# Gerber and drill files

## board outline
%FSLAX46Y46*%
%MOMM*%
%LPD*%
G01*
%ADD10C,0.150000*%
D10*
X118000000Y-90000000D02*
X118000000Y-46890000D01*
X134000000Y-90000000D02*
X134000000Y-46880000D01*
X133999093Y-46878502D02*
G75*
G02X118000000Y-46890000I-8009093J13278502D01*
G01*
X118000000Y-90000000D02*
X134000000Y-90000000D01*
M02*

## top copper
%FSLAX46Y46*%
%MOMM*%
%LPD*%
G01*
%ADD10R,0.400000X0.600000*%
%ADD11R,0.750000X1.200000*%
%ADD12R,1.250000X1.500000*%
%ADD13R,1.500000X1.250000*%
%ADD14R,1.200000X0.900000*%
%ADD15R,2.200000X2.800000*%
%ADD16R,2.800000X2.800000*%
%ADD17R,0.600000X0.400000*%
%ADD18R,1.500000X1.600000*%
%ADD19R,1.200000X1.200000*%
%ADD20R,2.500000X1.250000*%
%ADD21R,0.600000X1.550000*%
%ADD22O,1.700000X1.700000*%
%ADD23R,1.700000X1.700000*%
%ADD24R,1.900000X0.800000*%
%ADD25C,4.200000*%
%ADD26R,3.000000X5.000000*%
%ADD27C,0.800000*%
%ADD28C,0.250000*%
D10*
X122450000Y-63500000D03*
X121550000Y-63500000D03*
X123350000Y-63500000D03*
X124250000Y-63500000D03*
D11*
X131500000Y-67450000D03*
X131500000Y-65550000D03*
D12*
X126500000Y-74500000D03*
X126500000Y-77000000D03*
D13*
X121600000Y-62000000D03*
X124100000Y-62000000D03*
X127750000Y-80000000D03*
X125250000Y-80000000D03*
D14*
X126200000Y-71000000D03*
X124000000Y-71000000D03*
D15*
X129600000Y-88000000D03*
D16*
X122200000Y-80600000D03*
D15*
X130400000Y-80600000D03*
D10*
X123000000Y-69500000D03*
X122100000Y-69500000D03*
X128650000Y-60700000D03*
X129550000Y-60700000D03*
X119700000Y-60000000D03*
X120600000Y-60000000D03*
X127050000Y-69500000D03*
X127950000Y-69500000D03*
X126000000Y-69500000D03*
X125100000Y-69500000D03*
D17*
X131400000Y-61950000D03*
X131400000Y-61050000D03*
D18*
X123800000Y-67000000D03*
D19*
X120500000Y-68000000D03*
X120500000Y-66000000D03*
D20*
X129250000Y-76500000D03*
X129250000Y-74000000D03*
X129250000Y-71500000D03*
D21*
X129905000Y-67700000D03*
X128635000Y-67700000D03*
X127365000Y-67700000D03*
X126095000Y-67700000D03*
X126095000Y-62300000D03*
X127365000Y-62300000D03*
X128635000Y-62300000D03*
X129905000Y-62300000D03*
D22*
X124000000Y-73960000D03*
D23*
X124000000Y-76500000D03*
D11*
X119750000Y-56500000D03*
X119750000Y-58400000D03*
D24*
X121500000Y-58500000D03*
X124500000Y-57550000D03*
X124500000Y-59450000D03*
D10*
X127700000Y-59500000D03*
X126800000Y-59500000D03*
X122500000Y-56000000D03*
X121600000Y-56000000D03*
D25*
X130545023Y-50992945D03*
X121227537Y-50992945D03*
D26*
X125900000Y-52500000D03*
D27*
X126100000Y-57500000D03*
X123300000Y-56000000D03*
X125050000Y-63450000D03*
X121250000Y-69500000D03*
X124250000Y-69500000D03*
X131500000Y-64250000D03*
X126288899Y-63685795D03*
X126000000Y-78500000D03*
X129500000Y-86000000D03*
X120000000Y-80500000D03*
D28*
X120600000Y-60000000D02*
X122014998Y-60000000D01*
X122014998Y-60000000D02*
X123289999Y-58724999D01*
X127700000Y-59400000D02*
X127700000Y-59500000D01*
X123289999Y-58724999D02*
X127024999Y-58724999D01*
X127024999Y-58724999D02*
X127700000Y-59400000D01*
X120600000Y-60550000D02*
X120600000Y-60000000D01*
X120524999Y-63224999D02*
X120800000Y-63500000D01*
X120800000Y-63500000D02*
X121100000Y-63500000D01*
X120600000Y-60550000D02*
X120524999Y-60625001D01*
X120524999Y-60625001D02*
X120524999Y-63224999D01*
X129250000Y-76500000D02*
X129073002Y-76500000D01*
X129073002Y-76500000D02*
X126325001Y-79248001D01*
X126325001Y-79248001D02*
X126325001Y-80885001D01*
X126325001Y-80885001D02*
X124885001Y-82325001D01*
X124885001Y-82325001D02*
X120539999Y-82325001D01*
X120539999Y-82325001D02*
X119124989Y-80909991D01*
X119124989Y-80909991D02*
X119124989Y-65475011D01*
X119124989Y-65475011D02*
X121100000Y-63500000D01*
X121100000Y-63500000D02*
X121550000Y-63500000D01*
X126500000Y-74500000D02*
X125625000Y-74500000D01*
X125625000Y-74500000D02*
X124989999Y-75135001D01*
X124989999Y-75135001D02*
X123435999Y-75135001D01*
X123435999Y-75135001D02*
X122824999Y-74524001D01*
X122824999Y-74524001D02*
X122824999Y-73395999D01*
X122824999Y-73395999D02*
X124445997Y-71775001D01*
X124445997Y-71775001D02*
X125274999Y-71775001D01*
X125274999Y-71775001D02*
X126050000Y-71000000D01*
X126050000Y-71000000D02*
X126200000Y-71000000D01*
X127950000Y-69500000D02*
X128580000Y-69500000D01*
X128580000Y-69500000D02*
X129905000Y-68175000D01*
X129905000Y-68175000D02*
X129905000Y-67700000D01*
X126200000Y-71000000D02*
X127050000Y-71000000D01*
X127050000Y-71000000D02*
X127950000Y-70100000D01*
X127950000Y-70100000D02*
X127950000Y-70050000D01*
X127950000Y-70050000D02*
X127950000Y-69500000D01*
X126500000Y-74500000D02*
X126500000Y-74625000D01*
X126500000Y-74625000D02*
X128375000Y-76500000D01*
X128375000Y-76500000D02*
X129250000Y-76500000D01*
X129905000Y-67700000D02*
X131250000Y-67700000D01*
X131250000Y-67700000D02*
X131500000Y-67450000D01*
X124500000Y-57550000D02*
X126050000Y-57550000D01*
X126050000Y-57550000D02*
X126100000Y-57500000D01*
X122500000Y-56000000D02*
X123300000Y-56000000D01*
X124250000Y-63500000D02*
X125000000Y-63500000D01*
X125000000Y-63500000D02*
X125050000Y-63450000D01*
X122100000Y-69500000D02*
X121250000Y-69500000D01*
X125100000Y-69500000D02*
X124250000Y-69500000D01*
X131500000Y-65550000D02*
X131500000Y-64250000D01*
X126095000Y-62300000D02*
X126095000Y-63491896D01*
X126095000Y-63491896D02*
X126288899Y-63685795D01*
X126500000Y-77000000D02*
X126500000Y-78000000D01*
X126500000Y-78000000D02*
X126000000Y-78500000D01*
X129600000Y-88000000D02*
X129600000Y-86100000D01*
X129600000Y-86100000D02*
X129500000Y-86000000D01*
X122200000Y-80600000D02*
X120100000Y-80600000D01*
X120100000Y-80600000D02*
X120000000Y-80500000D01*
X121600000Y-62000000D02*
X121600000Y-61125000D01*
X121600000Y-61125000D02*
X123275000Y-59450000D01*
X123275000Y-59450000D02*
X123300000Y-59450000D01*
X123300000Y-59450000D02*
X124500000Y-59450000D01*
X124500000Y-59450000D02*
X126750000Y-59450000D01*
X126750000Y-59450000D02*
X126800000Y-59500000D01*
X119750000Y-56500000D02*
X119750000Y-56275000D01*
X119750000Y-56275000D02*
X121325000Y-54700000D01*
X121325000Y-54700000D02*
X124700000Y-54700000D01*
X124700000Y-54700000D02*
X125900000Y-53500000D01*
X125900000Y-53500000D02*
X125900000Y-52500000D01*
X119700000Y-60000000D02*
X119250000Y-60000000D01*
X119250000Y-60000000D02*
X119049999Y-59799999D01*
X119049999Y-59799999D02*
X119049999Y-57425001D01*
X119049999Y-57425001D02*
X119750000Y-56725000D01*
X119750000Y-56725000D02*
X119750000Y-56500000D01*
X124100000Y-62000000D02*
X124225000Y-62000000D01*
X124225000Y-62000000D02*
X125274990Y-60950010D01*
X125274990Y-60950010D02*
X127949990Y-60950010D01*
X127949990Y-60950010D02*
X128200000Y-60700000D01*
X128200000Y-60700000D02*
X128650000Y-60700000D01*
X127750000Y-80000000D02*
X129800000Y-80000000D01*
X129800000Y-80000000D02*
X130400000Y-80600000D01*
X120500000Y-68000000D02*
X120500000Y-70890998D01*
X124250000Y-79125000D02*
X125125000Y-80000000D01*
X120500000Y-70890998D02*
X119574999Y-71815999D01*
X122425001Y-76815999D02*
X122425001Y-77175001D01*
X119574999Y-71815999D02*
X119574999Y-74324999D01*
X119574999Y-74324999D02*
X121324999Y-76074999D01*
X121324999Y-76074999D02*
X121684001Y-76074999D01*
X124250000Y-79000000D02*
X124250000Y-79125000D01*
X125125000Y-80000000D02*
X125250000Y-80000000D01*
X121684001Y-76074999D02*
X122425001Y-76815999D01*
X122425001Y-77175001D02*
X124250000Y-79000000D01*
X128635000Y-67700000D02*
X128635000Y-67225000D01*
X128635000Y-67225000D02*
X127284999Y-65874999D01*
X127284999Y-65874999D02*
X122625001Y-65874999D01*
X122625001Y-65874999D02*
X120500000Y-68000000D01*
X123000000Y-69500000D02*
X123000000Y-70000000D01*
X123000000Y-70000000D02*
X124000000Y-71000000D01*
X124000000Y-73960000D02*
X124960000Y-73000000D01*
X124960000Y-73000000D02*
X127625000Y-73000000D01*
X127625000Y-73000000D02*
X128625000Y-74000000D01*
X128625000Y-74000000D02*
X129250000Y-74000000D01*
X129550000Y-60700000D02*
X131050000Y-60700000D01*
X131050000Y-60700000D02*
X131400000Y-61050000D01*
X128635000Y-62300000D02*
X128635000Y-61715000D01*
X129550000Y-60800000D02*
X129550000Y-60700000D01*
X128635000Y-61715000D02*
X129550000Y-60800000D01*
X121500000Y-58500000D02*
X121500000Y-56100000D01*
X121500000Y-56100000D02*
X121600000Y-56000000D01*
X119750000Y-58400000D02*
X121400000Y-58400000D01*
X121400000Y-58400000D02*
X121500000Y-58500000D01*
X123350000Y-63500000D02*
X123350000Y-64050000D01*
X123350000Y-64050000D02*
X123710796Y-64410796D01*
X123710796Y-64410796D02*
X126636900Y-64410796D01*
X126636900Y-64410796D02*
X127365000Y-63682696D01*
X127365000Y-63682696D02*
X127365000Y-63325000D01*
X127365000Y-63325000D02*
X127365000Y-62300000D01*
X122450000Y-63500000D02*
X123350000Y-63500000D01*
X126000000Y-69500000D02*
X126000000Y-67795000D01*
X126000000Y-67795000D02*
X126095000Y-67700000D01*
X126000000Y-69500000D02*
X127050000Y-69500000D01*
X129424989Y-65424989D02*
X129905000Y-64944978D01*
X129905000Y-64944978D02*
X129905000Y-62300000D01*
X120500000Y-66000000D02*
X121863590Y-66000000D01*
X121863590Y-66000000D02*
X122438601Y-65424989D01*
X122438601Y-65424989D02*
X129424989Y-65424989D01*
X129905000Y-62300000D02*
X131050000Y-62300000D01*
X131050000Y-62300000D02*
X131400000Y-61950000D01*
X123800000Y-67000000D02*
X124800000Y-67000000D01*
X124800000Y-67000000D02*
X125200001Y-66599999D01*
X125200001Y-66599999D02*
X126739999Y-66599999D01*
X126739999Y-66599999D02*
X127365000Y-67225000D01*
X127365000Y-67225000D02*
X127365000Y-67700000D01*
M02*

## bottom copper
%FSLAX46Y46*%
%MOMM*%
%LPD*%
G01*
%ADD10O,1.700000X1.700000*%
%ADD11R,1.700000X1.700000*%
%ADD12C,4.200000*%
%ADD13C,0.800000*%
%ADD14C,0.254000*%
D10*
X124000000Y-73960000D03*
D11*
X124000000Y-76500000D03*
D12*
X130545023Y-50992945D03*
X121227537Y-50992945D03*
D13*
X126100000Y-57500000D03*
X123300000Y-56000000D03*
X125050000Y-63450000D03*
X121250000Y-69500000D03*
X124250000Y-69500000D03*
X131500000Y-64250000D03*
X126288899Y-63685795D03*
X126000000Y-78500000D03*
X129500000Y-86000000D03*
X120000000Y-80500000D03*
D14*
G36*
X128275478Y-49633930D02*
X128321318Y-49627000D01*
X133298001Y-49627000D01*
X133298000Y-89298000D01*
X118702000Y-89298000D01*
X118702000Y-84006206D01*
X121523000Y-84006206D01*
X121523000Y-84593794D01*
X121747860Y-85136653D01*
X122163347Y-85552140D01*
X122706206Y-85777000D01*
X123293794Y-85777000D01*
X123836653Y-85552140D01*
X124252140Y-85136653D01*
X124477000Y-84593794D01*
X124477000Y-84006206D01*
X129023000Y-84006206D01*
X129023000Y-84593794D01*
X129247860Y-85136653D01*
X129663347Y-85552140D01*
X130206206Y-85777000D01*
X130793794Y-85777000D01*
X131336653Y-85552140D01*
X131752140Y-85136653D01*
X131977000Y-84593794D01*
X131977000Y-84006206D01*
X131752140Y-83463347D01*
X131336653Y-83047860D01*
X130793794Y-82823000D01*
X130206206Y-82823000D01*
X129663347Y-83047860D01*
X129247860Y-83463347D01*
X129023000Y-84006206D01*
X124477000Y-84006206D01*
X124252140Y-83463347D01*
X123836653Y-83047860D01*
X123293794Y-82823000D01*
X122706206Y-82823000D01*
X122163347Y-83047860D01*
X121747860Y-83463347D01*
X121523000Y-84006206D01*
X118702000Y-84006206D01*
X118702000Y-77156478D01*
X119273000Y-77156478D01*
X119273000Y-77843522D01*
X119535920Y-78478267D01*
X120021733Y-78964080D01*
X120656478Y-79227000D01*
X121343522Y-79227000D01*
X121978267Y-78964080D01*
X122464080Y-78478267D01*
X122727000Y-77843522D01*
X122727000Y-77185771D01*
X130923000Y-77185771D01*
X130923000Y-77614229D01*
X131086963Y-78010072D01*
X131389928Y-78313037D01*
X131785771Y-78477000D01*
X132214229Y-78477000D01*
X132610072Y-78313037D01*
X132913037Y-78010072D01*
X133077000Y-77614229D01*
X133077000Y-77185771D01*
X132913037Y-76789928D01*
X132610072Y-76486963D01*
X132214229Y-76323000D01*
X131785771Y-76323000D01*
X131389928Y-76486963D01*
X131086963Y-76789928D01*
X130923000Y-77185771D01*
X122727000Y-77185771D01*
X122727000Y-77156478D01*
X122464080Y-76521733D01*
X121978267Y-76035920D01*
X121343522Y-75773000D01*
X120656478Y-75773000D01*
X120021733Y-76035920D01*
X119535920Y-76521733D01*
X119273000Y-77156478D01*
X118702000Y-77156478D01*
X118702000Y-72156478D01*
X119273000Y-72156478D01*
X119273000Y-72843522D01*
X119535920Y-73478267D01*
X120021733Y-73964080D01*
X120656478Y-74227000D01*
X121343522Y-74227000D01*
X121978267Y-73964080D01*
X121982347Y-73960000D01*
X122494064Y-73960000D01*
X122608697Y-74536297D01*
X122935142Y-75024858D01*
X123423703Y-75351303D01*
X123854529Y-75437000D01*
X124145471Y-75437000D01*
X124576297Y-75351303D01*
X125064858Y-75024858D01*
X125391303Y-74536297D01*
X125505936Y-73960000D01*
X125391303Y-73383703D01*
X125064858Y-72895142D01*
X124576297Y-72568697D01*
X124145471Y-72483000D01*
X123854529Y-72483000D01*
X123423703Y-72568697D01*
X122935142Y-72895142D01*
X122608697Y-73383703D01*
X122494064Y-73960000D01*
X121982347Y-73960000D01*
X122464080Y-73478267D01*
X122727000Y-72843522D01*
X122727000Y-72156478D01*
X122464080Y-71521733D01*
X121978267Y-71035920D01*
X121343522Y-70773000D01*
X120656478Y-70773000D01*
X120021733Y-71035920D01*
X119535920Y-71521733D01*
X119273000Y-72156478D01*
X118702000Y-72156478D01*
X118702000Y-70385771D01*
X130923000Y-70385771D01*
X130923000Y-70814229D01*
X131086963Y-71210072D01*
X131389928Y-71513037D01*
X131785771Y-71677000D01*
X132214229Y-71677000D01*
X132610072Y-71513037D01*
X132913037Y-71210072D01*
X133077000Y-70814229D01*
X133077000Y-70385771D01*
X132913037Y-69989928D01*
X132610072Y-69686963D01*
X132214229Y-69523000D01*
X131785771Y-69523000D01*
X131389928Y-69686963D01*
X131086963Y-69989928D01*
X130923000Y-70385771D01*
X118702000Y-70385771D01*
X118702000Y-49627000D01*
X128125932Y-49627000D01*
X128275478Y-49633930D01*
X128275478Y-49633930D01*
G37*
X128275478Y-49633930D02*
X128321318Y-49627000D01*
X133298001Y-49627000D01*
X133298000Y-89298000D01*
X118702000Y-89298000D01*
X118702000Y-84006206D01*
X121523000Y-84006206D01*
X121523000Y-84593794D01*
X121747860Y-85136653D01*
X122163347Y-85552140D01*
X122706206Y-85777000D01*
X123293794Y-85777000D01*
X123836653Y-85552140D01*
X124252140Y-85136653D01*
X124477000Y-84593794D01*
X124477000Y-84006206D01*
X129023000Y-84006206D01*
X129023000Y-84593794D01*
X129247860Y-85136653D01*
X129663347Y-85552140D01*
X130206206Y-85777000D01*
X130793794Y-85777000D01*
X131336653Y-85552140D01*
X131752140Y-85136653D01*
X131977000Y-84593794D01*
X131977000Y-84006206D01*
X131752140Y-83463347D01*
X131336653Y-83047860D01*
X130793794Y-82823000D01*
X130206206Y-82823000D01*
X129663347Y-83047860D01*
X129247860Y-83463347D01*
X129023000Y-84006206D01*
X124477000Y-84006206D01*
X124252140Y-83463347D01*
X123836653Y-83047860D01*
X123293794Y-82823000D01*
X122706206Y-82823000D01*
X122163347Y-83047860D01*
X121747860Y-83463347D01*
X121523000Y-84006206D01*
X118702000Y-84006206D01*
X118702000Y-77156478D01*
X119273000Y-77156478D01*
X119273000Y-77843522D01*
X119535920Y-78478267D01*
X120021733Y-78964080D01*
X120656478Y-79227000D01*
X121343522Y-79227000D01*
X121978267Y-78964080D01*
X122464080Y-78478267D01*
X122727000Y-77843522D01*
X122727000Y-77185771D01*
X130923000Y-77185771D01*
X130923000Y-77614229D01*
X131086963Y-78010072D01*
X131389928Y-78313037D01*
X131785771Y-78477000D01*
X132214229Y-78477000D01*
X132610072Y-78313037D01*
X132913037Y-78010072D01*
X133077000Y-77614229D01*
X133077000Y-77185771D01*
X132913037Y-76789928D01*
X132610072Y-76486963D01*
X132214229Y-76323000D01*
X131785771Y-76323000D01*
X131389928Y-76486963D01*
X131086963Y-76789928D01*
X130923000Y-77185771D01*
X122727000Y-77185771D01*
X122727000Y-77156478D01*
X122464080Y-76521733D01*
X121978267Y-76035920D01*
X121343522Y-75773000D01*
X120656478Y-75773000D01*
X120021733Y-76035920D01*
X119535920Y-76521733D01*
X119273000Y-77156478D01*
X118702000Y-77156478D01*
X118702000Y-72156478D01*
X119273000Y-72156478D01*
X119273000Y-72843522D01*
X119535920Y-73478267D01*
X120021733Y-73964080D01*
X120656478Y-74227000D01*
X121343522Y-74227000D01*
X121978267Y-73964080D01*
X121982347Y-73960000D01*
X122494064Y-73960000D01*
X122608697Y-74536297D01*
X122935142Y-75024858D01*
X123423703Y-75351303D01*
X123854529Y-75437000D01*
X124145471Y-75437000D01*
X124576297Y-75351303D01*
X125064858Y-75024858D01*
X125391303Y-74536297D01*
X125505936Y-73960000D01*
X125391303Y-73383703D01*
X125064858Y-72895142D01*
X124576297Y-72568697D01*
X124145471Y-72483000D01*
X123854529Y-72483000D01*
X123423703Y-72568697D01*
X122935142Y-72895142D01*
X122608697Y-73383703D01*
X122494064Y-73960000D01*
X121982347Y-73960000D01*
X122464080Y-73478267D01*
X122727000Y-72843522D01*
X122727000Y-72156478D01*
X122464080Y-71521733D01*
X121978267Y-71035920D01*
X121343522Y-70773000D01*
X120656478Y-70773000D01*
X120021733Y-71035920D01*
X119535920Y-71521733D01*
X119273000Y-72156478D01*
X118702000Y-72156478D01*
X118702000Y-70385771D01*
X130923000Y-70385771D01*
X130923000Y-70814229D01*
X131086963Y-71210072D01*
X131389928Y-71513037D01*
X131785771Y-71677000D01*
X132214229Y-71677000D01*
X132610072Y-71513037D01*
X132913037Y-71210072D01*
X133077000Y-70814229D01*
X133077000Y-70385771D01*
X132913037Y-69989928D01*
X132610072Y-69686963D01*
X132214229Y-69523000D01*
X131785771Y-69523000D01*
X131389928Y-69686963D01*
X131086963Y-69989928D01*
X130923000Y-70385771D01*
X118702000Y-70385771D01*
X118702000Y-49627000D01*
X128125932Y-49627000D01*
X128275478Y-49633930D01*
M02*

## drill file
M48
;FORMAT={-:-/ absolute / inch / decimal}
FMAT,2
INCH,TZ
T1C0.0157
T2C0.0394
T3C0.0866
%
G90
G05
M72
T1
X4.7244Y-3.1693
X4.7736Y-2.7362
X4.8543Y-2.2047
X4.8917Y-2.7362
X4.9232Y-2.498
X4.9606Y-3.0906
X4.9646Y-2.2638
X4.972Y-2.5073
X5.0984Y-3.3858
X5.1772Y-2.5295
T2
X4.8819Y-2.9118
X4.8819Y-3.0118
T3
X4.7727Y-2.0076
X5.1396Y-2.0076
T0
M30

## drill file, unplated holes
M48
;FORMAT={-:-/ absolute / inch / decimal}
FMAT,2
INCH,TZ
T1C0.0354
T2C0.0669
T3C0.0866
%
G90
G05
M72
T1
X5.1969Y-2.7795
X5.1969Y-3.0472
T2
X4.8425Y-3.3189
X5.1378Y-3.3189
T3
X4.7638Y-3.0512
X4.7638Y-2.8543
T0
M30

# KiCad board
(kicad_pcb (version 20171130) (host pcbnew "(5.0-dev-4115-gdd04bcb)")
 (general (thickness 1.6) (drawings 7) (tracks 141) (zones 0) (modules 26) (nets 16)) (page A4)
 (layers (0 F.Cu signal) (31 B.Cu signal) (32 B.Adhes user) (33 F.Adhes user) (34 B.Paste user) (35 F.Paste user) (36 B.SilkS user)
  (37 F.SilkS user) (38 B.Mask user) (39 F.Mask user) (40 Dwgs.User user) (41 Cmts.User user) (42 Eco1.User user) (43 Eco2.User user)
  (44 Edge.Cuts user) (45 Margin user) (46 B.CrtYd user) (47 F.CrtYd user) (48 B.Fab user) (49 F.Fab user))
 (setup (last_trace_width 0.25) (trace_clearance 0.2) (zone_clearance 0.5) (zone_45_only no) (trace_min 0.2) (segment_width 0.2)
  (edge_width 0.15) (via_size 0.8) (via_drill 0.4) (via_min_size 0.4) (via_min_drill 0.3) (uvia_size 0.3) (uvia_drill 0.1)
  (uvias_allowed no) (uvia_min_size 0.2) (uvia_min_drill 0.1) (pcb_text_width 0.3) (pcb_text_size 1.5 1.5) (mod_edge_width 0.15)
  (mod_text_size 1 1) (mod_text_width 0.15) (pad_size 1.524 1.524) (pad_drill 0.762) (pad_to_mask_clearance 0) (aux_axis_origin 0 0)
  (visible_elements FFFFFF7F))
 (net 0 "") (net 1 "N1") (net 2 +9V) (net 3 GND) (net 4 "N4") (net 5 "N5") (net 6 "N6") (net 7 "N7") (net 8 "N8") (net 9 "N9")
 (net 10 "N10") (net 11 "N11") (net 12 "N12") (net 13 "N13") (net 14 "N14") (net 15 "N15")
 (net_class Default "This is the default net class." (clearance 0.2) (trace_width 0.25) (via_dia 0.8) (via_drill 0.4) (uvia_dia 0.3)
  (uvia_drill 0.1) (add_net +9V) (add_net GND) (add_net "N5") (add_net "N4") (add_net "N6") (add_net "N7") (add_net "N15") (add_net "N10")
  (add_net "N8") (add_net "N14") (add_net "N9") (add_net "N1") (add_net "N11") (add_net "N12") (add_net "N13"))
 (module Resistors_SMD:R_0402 (layer F.Cu) (at 122 63.5)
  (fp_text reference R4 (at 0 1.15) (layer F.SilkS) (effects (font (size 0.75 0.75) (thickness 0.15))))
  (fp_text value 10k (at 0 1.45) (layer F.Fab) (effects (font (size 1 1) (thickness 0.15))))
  (pad 2 smd rect (at 0.45 0) (size 0.4 0.6) (layers F.Cu F.Paste F.Mask) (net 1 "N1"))
  (pad 1 smd rect (at -0.45 0) (size 0.4 0.6) (layers F.Cu F.Paste F.Mask) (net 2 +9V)))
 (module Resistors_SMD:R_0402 (layer F.Cu) (at 123.8 63.5)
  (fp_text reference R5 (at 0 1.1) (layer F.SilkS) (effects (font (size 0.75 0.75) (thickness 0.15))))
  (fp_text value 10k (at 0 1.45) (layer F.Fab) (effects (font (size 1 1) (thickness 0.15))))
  (pad 1 smd rect (at -0.45 0) (size 0.4 0.6) (layers F.Cu F.Paste F.Mask) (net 1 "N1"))
  (pad 2 smd rect (at 0.45 0) (size 0.4 0.6) (layers F.Cu F.Paste F.Mask) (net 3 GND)))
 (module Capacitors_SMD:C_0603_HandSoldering (layer F.Cu) (at 131.5 66.5 270)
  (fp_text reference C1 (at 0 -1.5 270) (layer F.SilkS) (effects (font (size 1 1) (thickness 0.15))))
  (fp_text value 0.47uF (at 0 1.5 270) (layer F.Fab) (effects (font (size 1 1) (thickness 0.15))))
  (pad 2 smd rect (at 0.95 0 270) (size 1.2 0.75) (layers F.Cu F.Paste F.Mask) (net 2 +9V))
  (pad 1 smd rect (at -0.95 0 270) (size 1.2 0.75) (layers F.Cu F.Paste F.Mask) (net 3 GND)))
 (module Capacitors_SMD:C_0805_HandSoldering (layer F.Cu) (at 126.5 75.75 90)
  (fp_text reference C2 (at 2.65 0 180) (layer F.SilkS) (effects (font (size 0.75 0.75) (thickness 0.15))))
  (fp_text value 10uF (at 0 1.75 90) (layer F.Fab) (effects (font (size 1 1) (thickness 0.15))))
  (pad 2 smd rect (at 1.25 0 90) (size 1.5 1.25) (layers F.Cu F.Paste F.Mask) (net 2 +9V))
  (pad 1 smd rect (at -1.25 0 90) (size 1.5 1.25) (layers F.Cu F.Paste F.Mask) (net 3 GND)))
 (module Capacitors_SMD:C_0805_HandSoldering (layer F.Cu) (at 122.85 62 180)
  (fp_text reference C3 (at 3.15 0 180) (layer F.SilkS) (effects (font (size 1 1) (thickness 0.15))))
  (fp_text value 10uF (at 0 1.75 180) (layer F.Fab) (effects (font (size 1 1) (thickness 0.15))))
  (pad 2 smd rect (at 1.25 0 180) (size 1.5 1.25) (layers F.Cu F.Paste F.Mask) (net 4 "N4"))
  (pad 1 smd rect (at -1.25 0 180) (size 1.5 1.25) (layers F.Cu F.Paste F.Mask) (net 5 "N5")))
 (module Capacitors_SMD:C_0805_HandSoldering (layer F.Cu) (at 126.5 80 180)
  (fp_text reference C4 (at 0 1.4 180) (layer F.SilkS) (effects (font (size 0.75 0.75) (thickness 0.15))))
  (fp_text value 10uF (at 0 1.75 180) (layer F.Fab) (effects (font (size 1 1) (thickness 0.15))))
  (pad 1 smd rect (at -1.25 0 180) (size 1.5 1.25) (layers F.Cu F.Paste F.Mask) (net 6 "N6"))
  (pad 2 smd rect (at 1.25 0 180) (size 1.5 1.25) (layers F.Cu F.Paste F.Mask) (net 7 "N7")))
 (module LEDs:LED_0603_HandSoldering (layer F.Cu) (at 125.1 71)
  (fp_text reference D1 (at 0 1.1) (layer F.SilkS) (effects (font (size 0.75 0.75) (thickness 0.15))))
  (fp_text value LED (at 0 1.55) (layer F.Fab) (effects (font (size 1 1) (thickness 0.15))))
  (pad 2 smd rect (at 1.1 0) (size 1.2 0.9) (layers F.Cu F.Paste F.Mask) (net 2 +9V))
  (pad 1 smd rect (at -1.1 0) (size 1.2 0.9) (layers F.Cu F.Paste F.Mask) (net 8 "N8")))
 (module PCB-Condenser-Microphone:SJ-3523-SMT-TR (layer F.Cu) (at 126.5 84.3 270)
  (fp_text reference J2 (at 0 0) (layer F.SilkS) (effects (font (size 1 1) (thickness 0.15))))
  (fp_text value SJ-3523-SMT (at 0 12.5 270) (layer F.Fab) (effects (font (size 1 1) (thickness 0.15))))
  (pad "" np_thru_hole circle (at 0 3.5 270) (size 1.7 1.7) (drill 1.7) (layers *.Cu *.Mask))
  (pad "" np_thru_hole circle (at 0 -4 270) (size 1.7 1.7) (drill 1.7) (layers *.Cu *.Mask))
  (pad 1 smd rect (at 3.7 -3.1) (size 2.2 2.8) (layers F.Cu F.Paste F.Mask) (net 3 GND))
  (pad 3 smd rect (at -3.7 4.3 270) (size 2.8 2.8) (layers F.Cu F.Paste F.Mask) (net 3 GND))
  (pad 2 smd rect (at -3.7 -3.9) (size 2.2 2.8) (layers F.Cu F.Paste F.Mask) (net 6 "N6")))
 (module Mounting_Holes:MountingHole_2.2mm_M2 (layer F.Cu) (at 121 72.5)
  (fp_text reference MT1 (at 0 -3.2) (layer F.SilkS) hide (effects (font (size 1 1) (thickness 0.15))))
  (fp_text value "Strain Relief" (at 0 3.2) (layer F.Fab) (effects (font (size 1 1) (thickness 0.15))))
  (pad 1 np_thru_hole circle (at 0 0) (size 2.2 2.2) (drill 2.2) (layers *.Cu *.Mask)))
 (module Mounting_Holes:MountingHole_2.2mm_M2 (layer F.Cu) (at 121 77.5)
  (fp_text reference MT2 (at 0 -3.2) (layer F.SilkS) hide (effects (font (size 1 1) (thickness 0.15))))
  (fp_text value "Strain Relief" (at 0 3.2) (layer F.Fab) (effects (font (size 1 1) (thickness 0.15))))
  (pad 1 np_thru_hole circle (at 0 0) (size 2.2 2.2) (drill 2.2) (layers *.Cu *.Mask)))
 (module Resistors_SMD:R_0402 (layer F.Cu) (at 122.55 69.5 180)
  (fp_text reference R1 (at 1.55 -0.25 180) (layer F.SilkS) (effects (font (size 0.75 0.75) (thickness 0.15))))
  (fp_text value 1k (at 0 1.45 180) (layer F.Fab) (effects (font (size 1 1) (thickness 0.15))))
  (pad 1 smd rect (at -0.45 0 180) (size 0.4 0.6) (layers F.Cu F.Paste F.Mask) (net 8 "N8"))
  (pad 2 smd rect (at 0.45 0 180) (size 0.4 0.6) (layers F.Cu F.Paste F.Mask) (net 3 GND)))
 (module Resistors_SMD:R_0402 (layer F.Cu) (at 129.1 60.7 180)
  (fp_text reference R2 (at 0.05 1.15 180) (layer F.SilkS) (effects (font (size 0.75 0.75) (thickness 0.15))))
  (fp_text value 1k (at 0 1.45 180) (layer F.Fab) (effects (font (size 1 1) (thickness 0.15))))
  (pad 2 smd rect (at 0.45 0 180) (size 0.4 0.6) (layers F.Cu F.Paste F.Mask) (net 5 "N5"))
  (pad 1 smd rect (at -0.45 0 180) (size 0.4 0.6) (layers F.Cu F.Paste F.Mask) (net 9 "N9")))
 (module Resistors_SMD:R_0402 (layer F.Cu) (at 120.15 60 180)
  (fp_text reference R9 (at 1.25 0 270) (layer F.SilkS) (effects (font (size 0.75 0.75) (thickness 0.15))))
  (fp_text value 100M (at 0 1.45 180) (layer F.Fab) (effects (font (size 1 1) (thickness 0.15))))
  (pad 2 smd rect (at 0.45 0 180) (size 0.4 0.6) (layers F.Cu F.Paste F.Mask) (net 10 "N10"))
  (pad 1 smd rect (at -0.45 0 180) (size 0.4 0.6) (layers F.Cu F.Paste F.Mask) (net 2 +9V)))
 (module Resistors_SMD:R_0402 (layer F.Cu) (at 127.5 69.5 180)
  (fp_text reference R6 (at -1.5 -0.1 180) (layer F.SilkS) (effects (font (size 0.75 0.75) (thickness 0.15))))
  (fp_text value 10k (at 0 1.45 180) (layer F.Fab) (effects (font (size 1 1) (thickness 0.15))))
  (pad 2 smd rect (at 0.45 0 180) (size 0.4 0.6) (layers F.Cu F.Paste F.Mask) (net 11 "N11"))
  (pad 1 smd rect (at -0.45 0 180) (size 0.4 0.6) (layers F.Cu F.Paste F.Mask) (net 2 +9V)))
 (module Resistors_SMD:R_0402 (layer F.Cu) (at 125.55 69.5 180)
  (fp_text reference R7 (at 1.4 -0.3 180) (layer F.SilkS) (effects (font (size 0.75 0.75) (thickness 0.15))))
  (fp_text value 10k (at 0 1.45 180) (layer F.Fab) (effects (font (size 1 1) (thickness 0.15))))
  (pad 1 smd rect (at -0.45 0 180) (size 0.4 0.6) (layers F.Cu F.Paste F.Mask) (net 11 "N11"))
  (pad 2 smd rect (at 0.45 0 180) (size 0.4 0.6) (layers F.Cu F.Paste F.Mask) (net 3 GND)))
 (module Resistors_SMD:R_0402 (layer F.Cu) (at 131.4 61.5 90)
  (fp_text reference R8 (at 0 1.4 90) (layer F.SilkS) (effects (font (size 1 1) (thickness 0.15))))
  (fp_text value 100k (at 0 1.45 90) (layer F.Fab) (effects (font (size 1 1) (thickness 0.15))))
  (pad 1 smd rect (at -0.45 0 90) (size 0.4 0.6) (layers F.Cu F.Paste F.Mask) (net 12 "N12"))
  (pad 2 smd rect (at 0.45 0 90) (size 0.4 0.6) (layers F.Cu F.Paste F.Mask) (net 9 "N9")))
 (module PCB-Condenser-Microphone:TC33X (layer F.Cu) (at 122.3 67 270)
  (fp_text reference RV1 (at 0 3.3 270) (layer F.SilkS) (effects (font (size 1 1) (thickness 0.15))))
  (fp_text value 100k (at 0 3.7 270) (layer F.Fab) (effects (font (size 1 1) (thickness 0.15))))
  (pad 2 smd rect (at 0 -1.5 270) (size 1.6 1.5) (layers F.Cu F.Paste F.Mask) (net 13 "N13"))
  (pad 3 smd rect (at 1 1.8 270) (size 1.2 1.2) (layers F.Cu F.Paste F.Mask) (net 7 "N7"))
  (pad 1 smd rect (at -1 1.8 270) (size 1.2 1.2) (layers F.Cu F.Paste F.Mask) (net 12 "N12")))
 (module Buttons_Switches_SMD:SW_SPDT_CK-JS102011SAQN (layer F.Cu) (at 132 74 90)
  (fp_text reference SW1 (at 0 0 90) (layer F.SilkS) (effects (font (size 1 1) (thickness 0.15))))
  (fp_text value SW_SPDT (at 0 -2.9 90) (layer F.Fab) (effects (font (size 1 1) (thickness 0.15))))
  (pad 1 smd rect (at -2.5 -2.75 90) (size 1.25 2.5) (layers F.Cu F.Paste F.Mask) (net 2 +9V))
  (pad 2 smd rect (at 0 -2.75 90) (size 1.25 2.5) (layers F.Cu F.Paste F.Mask) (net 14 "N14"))
  (pad 3 smd rect (at 2.5 -2.75 90) (size 1.25 2.5) (layers F.Cu F.Paste F.Mask))
  (pad "" np_thru_hole circle (at -3.4 0 90) (size 0.9 0.9) (drill 0.9) (layers *.Cu *.Mask))
  (pad "" np_thru_hole circle (at 3.4 0 90) (size 0.9 0.9) (drill 0.9) (layers *.Cu *.Mask)))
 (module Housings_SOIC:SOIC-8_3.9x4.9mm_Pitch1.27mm (layer F.Cu) (at 128 65 270)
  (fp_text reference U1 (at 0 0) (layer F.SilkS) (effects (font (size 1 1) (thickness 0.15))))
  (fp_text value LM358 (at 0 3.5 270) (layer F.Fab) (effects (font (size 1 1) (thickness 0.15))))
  (pad 8 smd rect (at 2.7 -1.905 270) (size 1.55 0.6) (layers F.Cu F.Paste F.Mask) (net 2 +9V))
  (pad 7 smd rect (at 2.7 -0.635 270) (size 1.55 0.6) (layers F.Cu F.Paste F.Mask) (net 7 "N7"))
  (pad 6 smd rect (at 2.7 0.635 270) (size 1.55 0.6) (layers F.Cu F.Paste F.Mask) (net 13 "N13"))
  (pad 5 smd rect (at 2.7 1.905 270) (size 1.55 0.6) (layers F.Cu F.Paste F.Mask) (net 11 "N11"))
  (pad 4 smd rect (at -2.7 1.905 270) (size 1.55 0.6) (layers F.Cu F.Paste F.Mask) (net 3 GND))
  (pad 3 smd rect (at -2.7 0.635 270) (size 1.55 0.6) (layers F.Cu F.Paste F.Mask) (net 1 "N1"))
  (pad 2 smd rect (at -2.7 -0.635 270) (size 1.55 0.6) (layers F.Cu F.Paste F.Mask) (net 9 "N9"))
  (pad 1 smd rect (at -2.7 -1.905 270) (size 1.55 0.6) (layers F.Cu F.Paste F.Mask) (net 12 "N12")))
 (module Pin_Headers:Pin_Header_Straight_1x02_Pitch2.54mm (layer F.Cu) (at 124 76.5 180)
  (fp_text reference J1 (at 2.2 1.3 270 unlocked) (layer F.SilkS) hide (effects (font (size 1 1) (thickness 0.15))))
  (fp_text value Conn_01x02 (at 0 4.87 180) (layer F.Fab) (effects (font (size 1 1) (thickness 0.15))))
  (pad 2 thru_hole oval (at 0 2.54 180) (size 1.7 1.7) (drill 1) (layers *.Cu *.Mask) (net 14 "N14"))
  (pad 1 thru_hole rect (at 0 0 180) (size 1.7 1.7) (drill 1) (layers *.Cu *.Mask) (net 3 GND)))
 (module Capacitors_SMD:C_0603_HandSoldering (layer F.Cu) (at 119.75 57.45 90)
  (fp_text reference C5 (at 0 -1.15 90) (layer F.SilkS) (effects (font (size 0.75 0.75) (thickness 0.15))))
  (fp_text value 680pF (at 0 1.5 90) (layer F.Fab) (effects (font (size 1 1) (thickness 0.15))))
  (pad 2 smd rect (at 0.95 0 90) (size 1.2 0.75) (layers F.Cu F.Paste F.Mask) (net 10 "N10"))
  (pad 1 smd rect (at -0.95 0 90) (size 1.2 0.75) (layers F.Cu F.Paste F.Mask) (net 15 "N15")))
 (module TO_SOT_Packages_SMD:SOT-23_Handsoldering (layer F.Cu) (at 123 58.5 180)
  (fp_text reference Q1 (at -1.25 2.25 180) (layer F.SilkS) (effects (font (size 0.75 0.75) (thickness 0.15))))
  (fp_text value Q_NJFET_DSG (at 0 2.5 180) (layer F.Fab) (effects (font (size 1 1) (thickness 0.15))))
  (pad 3 smd rect (at 1.5 0 180) (size 1.9 0.8) (layers F.Cu F.Paste F.Mask) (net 15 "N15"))
  (pad 2 smd rect (at -1.5 0.95 180) (size 1.9 0.8) (layers F.Cu F.Paste F.Mask) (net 3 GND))
  (pad 1 smd rect (at -1.5 -0.95 180) (size 1.9 0.8) (layers F.Cu F.Paste F.Mask) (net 4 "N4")))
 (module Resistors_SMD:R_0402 (layer F.Cu) (at 127.25 59.5 180)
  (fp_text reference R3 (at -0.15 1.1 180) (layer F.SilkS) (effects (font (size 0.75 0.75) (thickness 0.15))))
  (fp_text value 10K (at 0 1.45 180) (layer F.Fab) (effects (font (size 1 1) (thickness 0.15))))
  (pad 1 smd rect (at -0.45 0 180) (size 0.4 0.6) (layers F.Cu F.Paste F.Mask) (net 2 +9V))
  (pad 2 smd rect (at 0.45 0 180) (size 0.4 0.6) (layers F.Cu F.Paste F.Mask) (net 4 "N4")))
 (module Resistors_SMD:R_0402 (layer F.Cu) (at 122.05 56)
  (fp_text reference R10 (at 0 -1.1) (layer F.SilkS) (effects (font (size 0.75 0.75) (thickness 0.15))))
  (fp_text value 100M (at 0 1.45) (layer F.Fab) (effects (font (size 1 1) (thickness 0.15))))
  (pad 2 smd rect (at 0.45 0) (size 0.4 0.6) (layers F.Cu F.Paste F.Mask) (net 3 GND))
  (pad 1 smd rect (at -0.45 0) (size 0.4 0.6) (layers F.Cu F.Paste F.Mask) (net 15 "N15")))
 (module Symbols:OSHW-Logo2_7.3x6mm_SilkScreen (layer B.Cu) (at 121.8 58.6 90)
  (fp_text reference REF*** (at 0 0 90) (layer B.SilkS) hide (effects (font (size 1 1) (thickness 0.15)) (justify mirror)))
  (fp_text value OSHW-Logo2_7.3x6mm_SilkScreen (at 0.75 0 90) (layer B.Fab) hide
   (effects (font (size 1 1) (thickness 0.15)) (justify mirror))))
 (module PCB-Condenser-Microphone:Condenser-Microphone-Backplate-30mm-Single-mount (layer F.Cu) (at 125.9 51)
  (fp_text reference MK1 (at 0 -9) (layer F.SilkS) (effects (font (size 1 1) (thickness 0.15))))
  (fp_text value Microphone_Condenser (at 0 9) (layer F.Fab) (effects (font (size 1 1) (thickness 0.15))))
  (pad 1 thru_hole circle (at 4.645023 -0.007055 285) (size 4.2 4.2) (drill 2.2) (layers *.Cu *.Mask) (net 3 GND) (clearance 1))
  (pad 1 thru_hole circle (at -4.672463 -0.007055 255) (size 4.2 4.2) (drill 2.2) (layers *.Cu *.Mask) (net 3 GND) (clearance 1))
  (pad 2 smd rect (at 0 1.5) (size 3 5) (layers F.Cu F.Paste F.Mask) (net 10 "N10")))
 (gr_line (start 118 90) (end 118 46.89) (layer Edge.Cuts) (width 0.15))
 (gr_line (start 134 90) (end 134 46.88) (layer Edge.Cuts) (width 0.15))
 (gr_arc (start 125.99 33.6) (end 118 46.89) (angle -62.11124932) (layer Edge.Cuts) (width 0.15))
 (gr_line (start 118 90) (end 134 90) (layer Edge.Cuts) (width 0.15))
 (segment (start 120.6 60) (end 122.014998 60) (width 0.25) (layer F.Cu) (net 2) (status 10))
 (segment (start 122.014998 60) (end 123.289999 58.724999) (width 0.25) (layer F.Cu) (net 2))
 (segment (start 127.7 59.4) (end 127.7 59.5) (width 0.25) (layer F.Cu) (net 2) (status 30))
 (segment (start 123.289999 58.724999) (end 127.024999 58.724999) (width 0.25) (layer F.Cu) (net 2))
 (segment (start 127.024999 58.724999) (end 127.7 59.4) (width 0.25) (layer F.Cu) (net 2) (status 20))
 (segment (start 120.6 60.55) (end 120.6 60) (width 0.25) (layer F.Cu) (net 2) (status 20))
 (segment (start 120.524999 63.224999) (end 120.8 63.5) (width 0.25) (layer F.Cu) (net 2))
 (segment (start 120.8 63.5) (end 121.1 63.5) (width 0.25) (layer F.Cu) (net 2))
 (segment (start 120.6 60.55) (end 120.524999 60.625001) (width 0.25) (layer F.Cu) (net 2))
 (segment (start 120.524999 60.625001) (end 120.524999 63.224999) (width 0.25) (layer F.Cu) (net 2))
 (segment (start 129.25 76.5) (end 129.073002 76.5) (width 0.25) (layer F.Cu) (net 2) (status 30))
 (segment (start 129.073002 76.5) (end 126.325001 79.248001) (width 0.25) (layer F.Cu) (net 2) (status 10))
 (segment (start 126.325001 79.248001) (end 126.325001 80.885001) (width 0.25) (layer F.Cu) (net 2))
 (segment (start 126.325001 80.885001) (end 124.885001 82.325001) (width 0.25) (layer F.Cu) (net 2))
 (segment (start 124.885001 82.325001) (end 120.539999 82.325001) (width 0.25) (layer F.Cu) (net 2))
 (segment (start 120.539999 82.325001) (end 119.124989 80.909991) (width 0.25) (layer F.Cu) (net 2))
 (segment (start 119.124989 80.909991) (end 119.124989 65.475011) (width 0.25) (layer F.Cu) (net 2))
 (segment (start 119.124989 65.475011) (end 121.1 63.5) (width 0.25) (layer F.Cu) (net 2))
 (segment (start 121.1 63.5) (end 121.55 63.5) (width 0.25) (layer F.Cu) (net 2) (status 20))
 (segment (start 126.5 74.5) (end 125.625 74.5) (width 0.25) (layer F.Cu) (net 2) (status 10))
 (segment (start 125.625 74.5) (end 124.989999 75.135001) (width 0.25) (layer F.Cu) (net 2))
 (segment (start 124.989999 75.135001) (end 123.435999 75.135001) (width 0.25) (layer F.Cu) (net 2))
 (segment (start 123.435999 75.135001) (end 122.824999 74.524001) (width 0.25) (layer F.Cu) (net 2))
 (segment (start 122.824999 74.524001) (end 122.824999 73.395999) (width 0.25) (layer F.Cu) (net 2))
 (segment (start 122.824999 73.395999) (end 124.445997 71.775001) (width 0.25) (layer F.Cu) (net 2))
 (segment (start 124.445997 71.775001) (end 125.274999 71.775001) (width 0.25) (layer F.Cu) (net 2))
 (segment (start 125.274999 71.775001) (end 126.05 71) (width 0.25) (layer F.Cu) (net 2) (status 20))
 (segment (start 126.05 71) (end 126.2 71) (width 0.25) (layer F.Cu) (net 2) (status 30))
 (segment (start 127.95 69.5) (end 128.58 69.5) (width 0.25) (layer F.Cu) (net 2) (status 10))
 (segment (start 128.58 69.5) (end 129.905 68.175) (width 0.25) (layer F.Cu) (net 2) (status 20))
 (segment (start 129.905 68.175) (end 129.905 67.7) (width 0.25) (layer F.Cu) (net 2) (status 30))
 (segment (start 126.2 71) (end 127.05 71) (width 0.25) (layer F.Cu) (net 2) (status 10))
 (segment (start 127.05 71) (end 127.95 70.1) (width 0.25) (layer F.Cu) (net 2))
 (segment (start 127.95 70.1) (end 127.95 70.05) (width 0.25) (layer F.Cu) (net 2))
 (segment (start 127.95 70.05) (end 127.95 69.5) (width 0.25) (layer F.Cu) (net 2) (status 20))
 (segment (start 126.5 74.5) (end 126.5 74.625) (width 0.25) (layer F.Cu) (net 2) (status 30))
 (segment (start 126.5 74.625) (end 128.375 76.5) (width 0.25) (layer F.Cu) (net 2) (status 30))
 (segment (start 128.375 76.5) (end 129.25 76.5) (width 0.25) (layer F.Cu) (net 2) (status 30))
 (segment (start 129.905 67.7) (end 131.25 67.7) (width 0.25) (layer F.Cu) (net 2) (status 30))
 (segment (start 131.25 67.7) (end 131.5 67.45) (width 0.25) (layer F.Cu) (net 2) (status 30))
 (segment (start 124.5 57.55) (end 126.05 57.55) (width 0.25) (layer F.Cu) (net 3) (status 10))
 (segment (start 126.05 57.55) (end 126.1 57.5) (width 0.25) (layer F.Cu) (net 3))
 (via (at 126.1 57.5) (size 0.8) (drill 0.4) (layers F.Cu B.Cu) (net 3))
 (segment (start 122.5 56) (end 123.3 56) (width 0.25) (layer F.Cu) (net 3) (status 10))
 (via (at 123.3 56) (size 0.8) (drill 0.4) (layers F.Cu B.Cu) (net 3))
 (segment (start 124.25 63.5) (end 125 63.5) (width 0.25) (layer F.Cu) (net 3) (status 10))
 (segment (start 125 63.5) (end 125.05 63.45) (width 0.25) (layer F.Cu) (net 3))
 (via (at 125.05 63.45) (size 0.8) (drill 0.4) (layers F.Cu B.Cu) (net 3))
 (segment (start 122.1 69.5) (end 121.25 69.5) (width 0.25) (layer F.Cu) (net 3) (status 10))
 (via (at 121.25 69.5) (size 0.8) (drill 0.4) (layers F.Cu B.Cu) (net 3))
 (segment (start 125.1 69.5) (end 124.25 69.5) (width 0.25) (layer F.Cu) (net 3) (status 10))
 (via (at 124.25 69.5) (size 0.8) (drill 0.4) (layers F.Cu B.Cu) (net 3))
 (segment (start 131.5 65.55) (end 131.5 64.25) (width 0.25) (layer F.Cu) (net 3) (status 10))
 (via (at 131.5 64.25) (size 0.8) (drill 0.4) (layers F.Cu B.Cu) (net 3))
 (segment (start 126.095 62.3) (end 126.095 63.491896) (width 0.25) (layer F.Cu) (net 3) (status 10))
 (segment (start 126.095 63.491896) (end 126.288899 63.685795) (width 0.25) (layer F.Cu) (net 3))
 (via (at 126.288899 63.685795) (size 0.8) (drill 0.4) (layers F.Cu B.Cu) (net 3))
 (segment (start 126.5 77) (end 126.5 78) (width 0.25) (layer F.Cu) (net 3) (status 10))
 (segment (start 126.5 78) (end 126 78.5) (width 0.25) (layer F.Cu) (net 3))
 (via (at 126 78.5) (size 0.8) (drill 0.4) (layers F.Cu B.Cu) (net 3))
 (segment (start 129.6 88) (end 129.6 86.1) (width 0.25) (layer F.Cu) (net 3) (status 10))
 (segment (start 129.6 86.1) (end 129.5 86) (width 0.25) (layer F.Cu) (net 3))
 (via (at 129.5 86) (size 0.8) (drill 0.4) (layers F.Cu B.Cu) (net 3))
 (segment (start 122.2 80.6) (end 120.1 80.6) (width 0.25) (layer F.Cu) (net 3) (status 10))
 (segment (start 120.1 80.6) (end 120 80.5) (width 0.25) (layer F.Cu) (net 3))
 (via (at 120 80.5) (size 0.8) (drill 0.4) (layers F.Cu B.Cu) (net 3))
 (segment (start 121.6 62) (end 121.6 61.125) (width 0.25) (layer F.Cu) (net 4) (status 10))
 (segment (start 121.6 61.125) (end 123.275 59.45) (width 0.25) (layer F.Cu) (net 4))
 (segment (start 123.275 59.45) (end 123.3 59.45) (width 0.25) (layer F.Cu) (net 4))
 (segment (start 123.3 59.45) (end 124.5 59.45) (width 0.25) (layer F.Cu) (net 4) (status 20))
 (segment (start 124.5 59.45) (end 126.75 59.45) (width 0.25) (layer F.Cu) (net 4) (status 30))
 (segment (start 126.75 59.45) (end 126.8 59.5) (width 0.25) (layer F.Cu) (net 4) (status 30))
 (segment (start 119.75 56.5) (end 119.75 56.275) (width 0.25) (layer F.Cu) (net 10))
 (segment (start 119.75 56.275) (end 121.325 54.7) (width 0.25) (layer F.Cu) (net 10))
 (segment (start 121.325 54.7) (end 124.7 54.7) (width 0.25) (layer F.Cu) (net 10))
 (segment (start 124.7 54.7) (end 125.9 53.5) (width 0.25) (layer F.Cu) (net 10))
 (segment (start 125.9 53.5) (end 125.9 52.5) (width 0.25) (layer F.Cu) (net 10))
 (segment (start 119.7 60) (end 119.25 60) (width 0.25) (layer F.Cu) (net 10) (status 10))
 (segment (start 119.25 60) (end 119.049999 59.799999) (width 0.25) (layer F.Cu) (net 10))
 (segment (start 119.049999 59.799999) (end 119.049999 57.425001) (width 0.25) (layer F.Cu) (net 10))
 (segment (start 119.049999 57.425001) (end 119.75 56.725) (width 0.25) (layer F.Cu) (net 10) (status 20))
 (segment (start 119.75 56.725) (end 119.75 56.5) (width 0.25) (layer F.Cu) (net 10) (status 30))
 (segment (start 124.1 62) (end 124.225 62) (width 0.25) (layer F.Cu) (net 5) (status 30))
 (segment (start 124.225 62) (end 125.27499 60.95001) (width 0.25) (layer F.Cu) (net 5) (status 10))
 (segment (start 125.27499 60.95001) (end 127.94999 60.95001) (width 0.25) (layer F.Cu) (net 5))
 (segment (start 127.94999 60.95001) (end 128.2 60.7) (width 0.25) (layer F.Cu) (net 5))
 (segment (start 128.2 60.7) (end 128.65 60.7) (width 0.25) (layer F.Cu) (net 5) (status 20))
 (segment (start 127.75 80) (end 129.8 80) (width 0.25) (layer F.Cu) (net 6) (status 30))
 (segment (start 129.8 80) (end 130.4 80.6) (width 0.25) (layer F.Cu) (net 6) (status 30))
 (segment (start 120.5 68) (end 120.5 70.890998) (width 0.25) (layer F.Cu) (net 7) (status 10))
 (segment (start 124.25 79.125) (end 125.125 80) (width 0.25) (layer F.Cu) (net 7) (status 20))
 (segment (start 120.5 70.890998) (end 119.574999 71.815999) (width 0.25) (layer F.Cu) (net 7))
 (segment (start 122.425001 76.815999) (end 122.425001 77.175001) (width 0.25) (layer F.Cu) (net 7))
 (segment (start 119.574999 71.815999) (end 119.574999 74.324999) (width 0.25) (layer F.Cu) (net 7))
 (segment (start 119.574999 74.324999) (end 121.324999 76.074999) (width 0.25) (layer F.Cu) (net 7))
 (segment (start 121.324999 76.074999) (end 121.684001 76.074999) (width 0.25) (layer F.Cu) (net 7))
 (segment (start 124.25 79) (end 124.25 79.125) (width 0.25) (layer F.Cu) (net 7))
 (segment (start 125.125 80) (end 125.25 80) (width 0.25) (layer F.Cu) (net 7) (status 30))
 (segment (start 121.684001 76.074999) (end 122.425001 76.815999) (width 0.25) (layer F.Cu) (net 7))
 (segment (start 122.425001 77.175001) (end 124.25 79) (width 0.25) (layer F.Cu) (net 7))
 (segment (start 128.635 67.7) (end 128.635 67.225) (width 0.25) (layer F.Cu) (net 7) (status 30))
 (segment (start 128.635 67.225) (end 127.284999 65.874999) (width 0.25) (layer F.Cu) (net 7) (status 10))
 (segment (start 127.284999 65.874999) (end 122.625001 65.874999) (width 0.25) (layer F.Cu) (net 7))
 (segment (start 122.625001 65.874999) (end 120.5 68) (width 0.25) (layer F.Cu) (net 7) (status 20))
 (segment (start 123 69.5) (end 123 70) (width 0.25) (layer F.Cu) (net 8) (status 10))
 (segment (start 123 70) (end 124 71) (width 0.25) (layer F.Cu) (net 8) (status 20))
 (segment (start 124 73.96) (end 124.96 73) (width 0.25) (layer F.Cu) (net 14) (status 10))
 (segment (start 124.96 73) (end 127.625 73) (width 0.25) (layer F.Cu) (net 14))
 (segment (start 127.625 73) (end 128.625 74) (width 0.25) (layer F.Cu) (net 14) (status 20))
 (segment (start 128.625 74) (end 129.25 74) (width 0.25) (layer F.Cu) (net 14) (status 30))
 (segment (start 129.55 60.7) (end 131.05 60.7) (width 0.25) (layer F.Cu) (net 9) (status 10))
 (segment (start 131.05 60.7) (end 131.4 61.05) (width 0.25) (layer F.Cu) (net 9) (status 20))
 (segment (start 128.635 62.3) (end 128.635 61.715) (width 0.25) (layer F.Cu) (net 9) (status 30))
 (segment (start 129.55 60.8) (end 129.55 60.7) (width 0.25) (layer F.Cu) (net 9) (status 30))
 (segment (start 128.635 61.715) (end 129.55 60.8) (width 0.25) (layer F.Cu) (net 9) (status 30))
 (segment (start 121.5 58.5) (end 121.5 56.1) (width 0.25) (layer F.Cu) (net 15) (status 30))
 (segment (start 121.5 56.1) (end 121.6 56) (width 0.25) (layer F.Cu) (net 15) (status 30))
 (segment (start 119.75 58.4) (end 121.4 58.4) (width 0.25) (layer F.Cu) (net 15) (status 30))
 (segment (start 121.4 58.4) (end 121.5 58.5) (width 0.25) (layer F.Cu) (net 15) (status 30))
 (segment (start 123.35 63.5) (end 123.35 64.05) (width 0.25) (layer F.Cu) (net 1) (status 10))
 (segment (start 123.35 64.05) (end 123.710796 64.410796) (width 0.25) (layer F.Cu) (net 1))
 (segment (start 123.710796 64.410796) (end 126.6369 64.410796) (width 0.25) (layer F.Cu) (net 1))
 (segment (start 126.6369 64.410796) (end 127.365 63.682696) (width 0.25) (layer F.Cu) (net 1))
 (segment (start 127.365 63.682696) (end 127.365 63.325) (width 0.25) (layer F.Cu) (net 1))
 (segment (start 127.365 63.325) (end 127.365 62.3) (width 0.25) (layer F.Cu) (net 1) (status 20))
 (segment (start 122.45 63.5) (end 123.35 63.5) (width 0.25) (layer F.Cu) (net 1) (status 30))
 (segment (start 126 69.5) (end 126 67.795) (width 0.25) (layer F.Cu) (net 11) (status 30))
 (segment (start 126 67.795) (end 126.095 67.7) (width 0.25) (layer F.Cu) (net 11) (status 30))
 (segment (start 126 69.5) (end 127.05 69.5) (width 0.25) (layer F.Cu) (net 11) (status 30))
 (segment (start 129.424989 65.424989) (end 129.905 64.944978) (width 0.25) (layer F.Cu) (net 12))
 (segment (start 129.905 64.944978) (end 129.905 62.3) (width 0.25) (layer F.Cu) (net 12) (status 20))
 (segment (start 120.5 66) (end 121.86359 66) (width 0.25) (layer F.Cu) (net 12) (status 10))
 (segment (start 121.86359 66) (end 122.438601 65.424989) (width 0.25) (layer F.Cu) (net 12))
 (segment (start 122.438601 65.424989) (end 129.424989 65.424989) (width 0.25) (layer F.Cu) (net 12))
 (segment (start 129.905 62.3) (end 131.05 62.3) (width 0.25) (layer F.Cu) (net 12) (status 10))
 (segment (start 131.05 62.3) (end 131.4 61.95) (width 0.25) (layer F.Cu) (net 12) (status 20))
 (segment (start 123.8 67) (end 124.8 67) (width 0.25) (layer F.Cu) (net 13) (status 10))
 (segment (start 124.8 67) (end 125.200001 66.599999) (width 0.25) (layer F.Cu) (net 13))
 (segment (start 125.200001 66.599999) (end 126.739999 66.599999) (width 0.25) (layer F.Cu) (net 13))
 (segment (start 126.739999 66.599999) (end 127.365 67.225) (width 0.25) (layer F.Cu) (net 13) (status 20))
 (segment (start 127.365 67.225) (end 127.365 67.7) (width 0.25) (layer F.Cu) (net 13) (status 30))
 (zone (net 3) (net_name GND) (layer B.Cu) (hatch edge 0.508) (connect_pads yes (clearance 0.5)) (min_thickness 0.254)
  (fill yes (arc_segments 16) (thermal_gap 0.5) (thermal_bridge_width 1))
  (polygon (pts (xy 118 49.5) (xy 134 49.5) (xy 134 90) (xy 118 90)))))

